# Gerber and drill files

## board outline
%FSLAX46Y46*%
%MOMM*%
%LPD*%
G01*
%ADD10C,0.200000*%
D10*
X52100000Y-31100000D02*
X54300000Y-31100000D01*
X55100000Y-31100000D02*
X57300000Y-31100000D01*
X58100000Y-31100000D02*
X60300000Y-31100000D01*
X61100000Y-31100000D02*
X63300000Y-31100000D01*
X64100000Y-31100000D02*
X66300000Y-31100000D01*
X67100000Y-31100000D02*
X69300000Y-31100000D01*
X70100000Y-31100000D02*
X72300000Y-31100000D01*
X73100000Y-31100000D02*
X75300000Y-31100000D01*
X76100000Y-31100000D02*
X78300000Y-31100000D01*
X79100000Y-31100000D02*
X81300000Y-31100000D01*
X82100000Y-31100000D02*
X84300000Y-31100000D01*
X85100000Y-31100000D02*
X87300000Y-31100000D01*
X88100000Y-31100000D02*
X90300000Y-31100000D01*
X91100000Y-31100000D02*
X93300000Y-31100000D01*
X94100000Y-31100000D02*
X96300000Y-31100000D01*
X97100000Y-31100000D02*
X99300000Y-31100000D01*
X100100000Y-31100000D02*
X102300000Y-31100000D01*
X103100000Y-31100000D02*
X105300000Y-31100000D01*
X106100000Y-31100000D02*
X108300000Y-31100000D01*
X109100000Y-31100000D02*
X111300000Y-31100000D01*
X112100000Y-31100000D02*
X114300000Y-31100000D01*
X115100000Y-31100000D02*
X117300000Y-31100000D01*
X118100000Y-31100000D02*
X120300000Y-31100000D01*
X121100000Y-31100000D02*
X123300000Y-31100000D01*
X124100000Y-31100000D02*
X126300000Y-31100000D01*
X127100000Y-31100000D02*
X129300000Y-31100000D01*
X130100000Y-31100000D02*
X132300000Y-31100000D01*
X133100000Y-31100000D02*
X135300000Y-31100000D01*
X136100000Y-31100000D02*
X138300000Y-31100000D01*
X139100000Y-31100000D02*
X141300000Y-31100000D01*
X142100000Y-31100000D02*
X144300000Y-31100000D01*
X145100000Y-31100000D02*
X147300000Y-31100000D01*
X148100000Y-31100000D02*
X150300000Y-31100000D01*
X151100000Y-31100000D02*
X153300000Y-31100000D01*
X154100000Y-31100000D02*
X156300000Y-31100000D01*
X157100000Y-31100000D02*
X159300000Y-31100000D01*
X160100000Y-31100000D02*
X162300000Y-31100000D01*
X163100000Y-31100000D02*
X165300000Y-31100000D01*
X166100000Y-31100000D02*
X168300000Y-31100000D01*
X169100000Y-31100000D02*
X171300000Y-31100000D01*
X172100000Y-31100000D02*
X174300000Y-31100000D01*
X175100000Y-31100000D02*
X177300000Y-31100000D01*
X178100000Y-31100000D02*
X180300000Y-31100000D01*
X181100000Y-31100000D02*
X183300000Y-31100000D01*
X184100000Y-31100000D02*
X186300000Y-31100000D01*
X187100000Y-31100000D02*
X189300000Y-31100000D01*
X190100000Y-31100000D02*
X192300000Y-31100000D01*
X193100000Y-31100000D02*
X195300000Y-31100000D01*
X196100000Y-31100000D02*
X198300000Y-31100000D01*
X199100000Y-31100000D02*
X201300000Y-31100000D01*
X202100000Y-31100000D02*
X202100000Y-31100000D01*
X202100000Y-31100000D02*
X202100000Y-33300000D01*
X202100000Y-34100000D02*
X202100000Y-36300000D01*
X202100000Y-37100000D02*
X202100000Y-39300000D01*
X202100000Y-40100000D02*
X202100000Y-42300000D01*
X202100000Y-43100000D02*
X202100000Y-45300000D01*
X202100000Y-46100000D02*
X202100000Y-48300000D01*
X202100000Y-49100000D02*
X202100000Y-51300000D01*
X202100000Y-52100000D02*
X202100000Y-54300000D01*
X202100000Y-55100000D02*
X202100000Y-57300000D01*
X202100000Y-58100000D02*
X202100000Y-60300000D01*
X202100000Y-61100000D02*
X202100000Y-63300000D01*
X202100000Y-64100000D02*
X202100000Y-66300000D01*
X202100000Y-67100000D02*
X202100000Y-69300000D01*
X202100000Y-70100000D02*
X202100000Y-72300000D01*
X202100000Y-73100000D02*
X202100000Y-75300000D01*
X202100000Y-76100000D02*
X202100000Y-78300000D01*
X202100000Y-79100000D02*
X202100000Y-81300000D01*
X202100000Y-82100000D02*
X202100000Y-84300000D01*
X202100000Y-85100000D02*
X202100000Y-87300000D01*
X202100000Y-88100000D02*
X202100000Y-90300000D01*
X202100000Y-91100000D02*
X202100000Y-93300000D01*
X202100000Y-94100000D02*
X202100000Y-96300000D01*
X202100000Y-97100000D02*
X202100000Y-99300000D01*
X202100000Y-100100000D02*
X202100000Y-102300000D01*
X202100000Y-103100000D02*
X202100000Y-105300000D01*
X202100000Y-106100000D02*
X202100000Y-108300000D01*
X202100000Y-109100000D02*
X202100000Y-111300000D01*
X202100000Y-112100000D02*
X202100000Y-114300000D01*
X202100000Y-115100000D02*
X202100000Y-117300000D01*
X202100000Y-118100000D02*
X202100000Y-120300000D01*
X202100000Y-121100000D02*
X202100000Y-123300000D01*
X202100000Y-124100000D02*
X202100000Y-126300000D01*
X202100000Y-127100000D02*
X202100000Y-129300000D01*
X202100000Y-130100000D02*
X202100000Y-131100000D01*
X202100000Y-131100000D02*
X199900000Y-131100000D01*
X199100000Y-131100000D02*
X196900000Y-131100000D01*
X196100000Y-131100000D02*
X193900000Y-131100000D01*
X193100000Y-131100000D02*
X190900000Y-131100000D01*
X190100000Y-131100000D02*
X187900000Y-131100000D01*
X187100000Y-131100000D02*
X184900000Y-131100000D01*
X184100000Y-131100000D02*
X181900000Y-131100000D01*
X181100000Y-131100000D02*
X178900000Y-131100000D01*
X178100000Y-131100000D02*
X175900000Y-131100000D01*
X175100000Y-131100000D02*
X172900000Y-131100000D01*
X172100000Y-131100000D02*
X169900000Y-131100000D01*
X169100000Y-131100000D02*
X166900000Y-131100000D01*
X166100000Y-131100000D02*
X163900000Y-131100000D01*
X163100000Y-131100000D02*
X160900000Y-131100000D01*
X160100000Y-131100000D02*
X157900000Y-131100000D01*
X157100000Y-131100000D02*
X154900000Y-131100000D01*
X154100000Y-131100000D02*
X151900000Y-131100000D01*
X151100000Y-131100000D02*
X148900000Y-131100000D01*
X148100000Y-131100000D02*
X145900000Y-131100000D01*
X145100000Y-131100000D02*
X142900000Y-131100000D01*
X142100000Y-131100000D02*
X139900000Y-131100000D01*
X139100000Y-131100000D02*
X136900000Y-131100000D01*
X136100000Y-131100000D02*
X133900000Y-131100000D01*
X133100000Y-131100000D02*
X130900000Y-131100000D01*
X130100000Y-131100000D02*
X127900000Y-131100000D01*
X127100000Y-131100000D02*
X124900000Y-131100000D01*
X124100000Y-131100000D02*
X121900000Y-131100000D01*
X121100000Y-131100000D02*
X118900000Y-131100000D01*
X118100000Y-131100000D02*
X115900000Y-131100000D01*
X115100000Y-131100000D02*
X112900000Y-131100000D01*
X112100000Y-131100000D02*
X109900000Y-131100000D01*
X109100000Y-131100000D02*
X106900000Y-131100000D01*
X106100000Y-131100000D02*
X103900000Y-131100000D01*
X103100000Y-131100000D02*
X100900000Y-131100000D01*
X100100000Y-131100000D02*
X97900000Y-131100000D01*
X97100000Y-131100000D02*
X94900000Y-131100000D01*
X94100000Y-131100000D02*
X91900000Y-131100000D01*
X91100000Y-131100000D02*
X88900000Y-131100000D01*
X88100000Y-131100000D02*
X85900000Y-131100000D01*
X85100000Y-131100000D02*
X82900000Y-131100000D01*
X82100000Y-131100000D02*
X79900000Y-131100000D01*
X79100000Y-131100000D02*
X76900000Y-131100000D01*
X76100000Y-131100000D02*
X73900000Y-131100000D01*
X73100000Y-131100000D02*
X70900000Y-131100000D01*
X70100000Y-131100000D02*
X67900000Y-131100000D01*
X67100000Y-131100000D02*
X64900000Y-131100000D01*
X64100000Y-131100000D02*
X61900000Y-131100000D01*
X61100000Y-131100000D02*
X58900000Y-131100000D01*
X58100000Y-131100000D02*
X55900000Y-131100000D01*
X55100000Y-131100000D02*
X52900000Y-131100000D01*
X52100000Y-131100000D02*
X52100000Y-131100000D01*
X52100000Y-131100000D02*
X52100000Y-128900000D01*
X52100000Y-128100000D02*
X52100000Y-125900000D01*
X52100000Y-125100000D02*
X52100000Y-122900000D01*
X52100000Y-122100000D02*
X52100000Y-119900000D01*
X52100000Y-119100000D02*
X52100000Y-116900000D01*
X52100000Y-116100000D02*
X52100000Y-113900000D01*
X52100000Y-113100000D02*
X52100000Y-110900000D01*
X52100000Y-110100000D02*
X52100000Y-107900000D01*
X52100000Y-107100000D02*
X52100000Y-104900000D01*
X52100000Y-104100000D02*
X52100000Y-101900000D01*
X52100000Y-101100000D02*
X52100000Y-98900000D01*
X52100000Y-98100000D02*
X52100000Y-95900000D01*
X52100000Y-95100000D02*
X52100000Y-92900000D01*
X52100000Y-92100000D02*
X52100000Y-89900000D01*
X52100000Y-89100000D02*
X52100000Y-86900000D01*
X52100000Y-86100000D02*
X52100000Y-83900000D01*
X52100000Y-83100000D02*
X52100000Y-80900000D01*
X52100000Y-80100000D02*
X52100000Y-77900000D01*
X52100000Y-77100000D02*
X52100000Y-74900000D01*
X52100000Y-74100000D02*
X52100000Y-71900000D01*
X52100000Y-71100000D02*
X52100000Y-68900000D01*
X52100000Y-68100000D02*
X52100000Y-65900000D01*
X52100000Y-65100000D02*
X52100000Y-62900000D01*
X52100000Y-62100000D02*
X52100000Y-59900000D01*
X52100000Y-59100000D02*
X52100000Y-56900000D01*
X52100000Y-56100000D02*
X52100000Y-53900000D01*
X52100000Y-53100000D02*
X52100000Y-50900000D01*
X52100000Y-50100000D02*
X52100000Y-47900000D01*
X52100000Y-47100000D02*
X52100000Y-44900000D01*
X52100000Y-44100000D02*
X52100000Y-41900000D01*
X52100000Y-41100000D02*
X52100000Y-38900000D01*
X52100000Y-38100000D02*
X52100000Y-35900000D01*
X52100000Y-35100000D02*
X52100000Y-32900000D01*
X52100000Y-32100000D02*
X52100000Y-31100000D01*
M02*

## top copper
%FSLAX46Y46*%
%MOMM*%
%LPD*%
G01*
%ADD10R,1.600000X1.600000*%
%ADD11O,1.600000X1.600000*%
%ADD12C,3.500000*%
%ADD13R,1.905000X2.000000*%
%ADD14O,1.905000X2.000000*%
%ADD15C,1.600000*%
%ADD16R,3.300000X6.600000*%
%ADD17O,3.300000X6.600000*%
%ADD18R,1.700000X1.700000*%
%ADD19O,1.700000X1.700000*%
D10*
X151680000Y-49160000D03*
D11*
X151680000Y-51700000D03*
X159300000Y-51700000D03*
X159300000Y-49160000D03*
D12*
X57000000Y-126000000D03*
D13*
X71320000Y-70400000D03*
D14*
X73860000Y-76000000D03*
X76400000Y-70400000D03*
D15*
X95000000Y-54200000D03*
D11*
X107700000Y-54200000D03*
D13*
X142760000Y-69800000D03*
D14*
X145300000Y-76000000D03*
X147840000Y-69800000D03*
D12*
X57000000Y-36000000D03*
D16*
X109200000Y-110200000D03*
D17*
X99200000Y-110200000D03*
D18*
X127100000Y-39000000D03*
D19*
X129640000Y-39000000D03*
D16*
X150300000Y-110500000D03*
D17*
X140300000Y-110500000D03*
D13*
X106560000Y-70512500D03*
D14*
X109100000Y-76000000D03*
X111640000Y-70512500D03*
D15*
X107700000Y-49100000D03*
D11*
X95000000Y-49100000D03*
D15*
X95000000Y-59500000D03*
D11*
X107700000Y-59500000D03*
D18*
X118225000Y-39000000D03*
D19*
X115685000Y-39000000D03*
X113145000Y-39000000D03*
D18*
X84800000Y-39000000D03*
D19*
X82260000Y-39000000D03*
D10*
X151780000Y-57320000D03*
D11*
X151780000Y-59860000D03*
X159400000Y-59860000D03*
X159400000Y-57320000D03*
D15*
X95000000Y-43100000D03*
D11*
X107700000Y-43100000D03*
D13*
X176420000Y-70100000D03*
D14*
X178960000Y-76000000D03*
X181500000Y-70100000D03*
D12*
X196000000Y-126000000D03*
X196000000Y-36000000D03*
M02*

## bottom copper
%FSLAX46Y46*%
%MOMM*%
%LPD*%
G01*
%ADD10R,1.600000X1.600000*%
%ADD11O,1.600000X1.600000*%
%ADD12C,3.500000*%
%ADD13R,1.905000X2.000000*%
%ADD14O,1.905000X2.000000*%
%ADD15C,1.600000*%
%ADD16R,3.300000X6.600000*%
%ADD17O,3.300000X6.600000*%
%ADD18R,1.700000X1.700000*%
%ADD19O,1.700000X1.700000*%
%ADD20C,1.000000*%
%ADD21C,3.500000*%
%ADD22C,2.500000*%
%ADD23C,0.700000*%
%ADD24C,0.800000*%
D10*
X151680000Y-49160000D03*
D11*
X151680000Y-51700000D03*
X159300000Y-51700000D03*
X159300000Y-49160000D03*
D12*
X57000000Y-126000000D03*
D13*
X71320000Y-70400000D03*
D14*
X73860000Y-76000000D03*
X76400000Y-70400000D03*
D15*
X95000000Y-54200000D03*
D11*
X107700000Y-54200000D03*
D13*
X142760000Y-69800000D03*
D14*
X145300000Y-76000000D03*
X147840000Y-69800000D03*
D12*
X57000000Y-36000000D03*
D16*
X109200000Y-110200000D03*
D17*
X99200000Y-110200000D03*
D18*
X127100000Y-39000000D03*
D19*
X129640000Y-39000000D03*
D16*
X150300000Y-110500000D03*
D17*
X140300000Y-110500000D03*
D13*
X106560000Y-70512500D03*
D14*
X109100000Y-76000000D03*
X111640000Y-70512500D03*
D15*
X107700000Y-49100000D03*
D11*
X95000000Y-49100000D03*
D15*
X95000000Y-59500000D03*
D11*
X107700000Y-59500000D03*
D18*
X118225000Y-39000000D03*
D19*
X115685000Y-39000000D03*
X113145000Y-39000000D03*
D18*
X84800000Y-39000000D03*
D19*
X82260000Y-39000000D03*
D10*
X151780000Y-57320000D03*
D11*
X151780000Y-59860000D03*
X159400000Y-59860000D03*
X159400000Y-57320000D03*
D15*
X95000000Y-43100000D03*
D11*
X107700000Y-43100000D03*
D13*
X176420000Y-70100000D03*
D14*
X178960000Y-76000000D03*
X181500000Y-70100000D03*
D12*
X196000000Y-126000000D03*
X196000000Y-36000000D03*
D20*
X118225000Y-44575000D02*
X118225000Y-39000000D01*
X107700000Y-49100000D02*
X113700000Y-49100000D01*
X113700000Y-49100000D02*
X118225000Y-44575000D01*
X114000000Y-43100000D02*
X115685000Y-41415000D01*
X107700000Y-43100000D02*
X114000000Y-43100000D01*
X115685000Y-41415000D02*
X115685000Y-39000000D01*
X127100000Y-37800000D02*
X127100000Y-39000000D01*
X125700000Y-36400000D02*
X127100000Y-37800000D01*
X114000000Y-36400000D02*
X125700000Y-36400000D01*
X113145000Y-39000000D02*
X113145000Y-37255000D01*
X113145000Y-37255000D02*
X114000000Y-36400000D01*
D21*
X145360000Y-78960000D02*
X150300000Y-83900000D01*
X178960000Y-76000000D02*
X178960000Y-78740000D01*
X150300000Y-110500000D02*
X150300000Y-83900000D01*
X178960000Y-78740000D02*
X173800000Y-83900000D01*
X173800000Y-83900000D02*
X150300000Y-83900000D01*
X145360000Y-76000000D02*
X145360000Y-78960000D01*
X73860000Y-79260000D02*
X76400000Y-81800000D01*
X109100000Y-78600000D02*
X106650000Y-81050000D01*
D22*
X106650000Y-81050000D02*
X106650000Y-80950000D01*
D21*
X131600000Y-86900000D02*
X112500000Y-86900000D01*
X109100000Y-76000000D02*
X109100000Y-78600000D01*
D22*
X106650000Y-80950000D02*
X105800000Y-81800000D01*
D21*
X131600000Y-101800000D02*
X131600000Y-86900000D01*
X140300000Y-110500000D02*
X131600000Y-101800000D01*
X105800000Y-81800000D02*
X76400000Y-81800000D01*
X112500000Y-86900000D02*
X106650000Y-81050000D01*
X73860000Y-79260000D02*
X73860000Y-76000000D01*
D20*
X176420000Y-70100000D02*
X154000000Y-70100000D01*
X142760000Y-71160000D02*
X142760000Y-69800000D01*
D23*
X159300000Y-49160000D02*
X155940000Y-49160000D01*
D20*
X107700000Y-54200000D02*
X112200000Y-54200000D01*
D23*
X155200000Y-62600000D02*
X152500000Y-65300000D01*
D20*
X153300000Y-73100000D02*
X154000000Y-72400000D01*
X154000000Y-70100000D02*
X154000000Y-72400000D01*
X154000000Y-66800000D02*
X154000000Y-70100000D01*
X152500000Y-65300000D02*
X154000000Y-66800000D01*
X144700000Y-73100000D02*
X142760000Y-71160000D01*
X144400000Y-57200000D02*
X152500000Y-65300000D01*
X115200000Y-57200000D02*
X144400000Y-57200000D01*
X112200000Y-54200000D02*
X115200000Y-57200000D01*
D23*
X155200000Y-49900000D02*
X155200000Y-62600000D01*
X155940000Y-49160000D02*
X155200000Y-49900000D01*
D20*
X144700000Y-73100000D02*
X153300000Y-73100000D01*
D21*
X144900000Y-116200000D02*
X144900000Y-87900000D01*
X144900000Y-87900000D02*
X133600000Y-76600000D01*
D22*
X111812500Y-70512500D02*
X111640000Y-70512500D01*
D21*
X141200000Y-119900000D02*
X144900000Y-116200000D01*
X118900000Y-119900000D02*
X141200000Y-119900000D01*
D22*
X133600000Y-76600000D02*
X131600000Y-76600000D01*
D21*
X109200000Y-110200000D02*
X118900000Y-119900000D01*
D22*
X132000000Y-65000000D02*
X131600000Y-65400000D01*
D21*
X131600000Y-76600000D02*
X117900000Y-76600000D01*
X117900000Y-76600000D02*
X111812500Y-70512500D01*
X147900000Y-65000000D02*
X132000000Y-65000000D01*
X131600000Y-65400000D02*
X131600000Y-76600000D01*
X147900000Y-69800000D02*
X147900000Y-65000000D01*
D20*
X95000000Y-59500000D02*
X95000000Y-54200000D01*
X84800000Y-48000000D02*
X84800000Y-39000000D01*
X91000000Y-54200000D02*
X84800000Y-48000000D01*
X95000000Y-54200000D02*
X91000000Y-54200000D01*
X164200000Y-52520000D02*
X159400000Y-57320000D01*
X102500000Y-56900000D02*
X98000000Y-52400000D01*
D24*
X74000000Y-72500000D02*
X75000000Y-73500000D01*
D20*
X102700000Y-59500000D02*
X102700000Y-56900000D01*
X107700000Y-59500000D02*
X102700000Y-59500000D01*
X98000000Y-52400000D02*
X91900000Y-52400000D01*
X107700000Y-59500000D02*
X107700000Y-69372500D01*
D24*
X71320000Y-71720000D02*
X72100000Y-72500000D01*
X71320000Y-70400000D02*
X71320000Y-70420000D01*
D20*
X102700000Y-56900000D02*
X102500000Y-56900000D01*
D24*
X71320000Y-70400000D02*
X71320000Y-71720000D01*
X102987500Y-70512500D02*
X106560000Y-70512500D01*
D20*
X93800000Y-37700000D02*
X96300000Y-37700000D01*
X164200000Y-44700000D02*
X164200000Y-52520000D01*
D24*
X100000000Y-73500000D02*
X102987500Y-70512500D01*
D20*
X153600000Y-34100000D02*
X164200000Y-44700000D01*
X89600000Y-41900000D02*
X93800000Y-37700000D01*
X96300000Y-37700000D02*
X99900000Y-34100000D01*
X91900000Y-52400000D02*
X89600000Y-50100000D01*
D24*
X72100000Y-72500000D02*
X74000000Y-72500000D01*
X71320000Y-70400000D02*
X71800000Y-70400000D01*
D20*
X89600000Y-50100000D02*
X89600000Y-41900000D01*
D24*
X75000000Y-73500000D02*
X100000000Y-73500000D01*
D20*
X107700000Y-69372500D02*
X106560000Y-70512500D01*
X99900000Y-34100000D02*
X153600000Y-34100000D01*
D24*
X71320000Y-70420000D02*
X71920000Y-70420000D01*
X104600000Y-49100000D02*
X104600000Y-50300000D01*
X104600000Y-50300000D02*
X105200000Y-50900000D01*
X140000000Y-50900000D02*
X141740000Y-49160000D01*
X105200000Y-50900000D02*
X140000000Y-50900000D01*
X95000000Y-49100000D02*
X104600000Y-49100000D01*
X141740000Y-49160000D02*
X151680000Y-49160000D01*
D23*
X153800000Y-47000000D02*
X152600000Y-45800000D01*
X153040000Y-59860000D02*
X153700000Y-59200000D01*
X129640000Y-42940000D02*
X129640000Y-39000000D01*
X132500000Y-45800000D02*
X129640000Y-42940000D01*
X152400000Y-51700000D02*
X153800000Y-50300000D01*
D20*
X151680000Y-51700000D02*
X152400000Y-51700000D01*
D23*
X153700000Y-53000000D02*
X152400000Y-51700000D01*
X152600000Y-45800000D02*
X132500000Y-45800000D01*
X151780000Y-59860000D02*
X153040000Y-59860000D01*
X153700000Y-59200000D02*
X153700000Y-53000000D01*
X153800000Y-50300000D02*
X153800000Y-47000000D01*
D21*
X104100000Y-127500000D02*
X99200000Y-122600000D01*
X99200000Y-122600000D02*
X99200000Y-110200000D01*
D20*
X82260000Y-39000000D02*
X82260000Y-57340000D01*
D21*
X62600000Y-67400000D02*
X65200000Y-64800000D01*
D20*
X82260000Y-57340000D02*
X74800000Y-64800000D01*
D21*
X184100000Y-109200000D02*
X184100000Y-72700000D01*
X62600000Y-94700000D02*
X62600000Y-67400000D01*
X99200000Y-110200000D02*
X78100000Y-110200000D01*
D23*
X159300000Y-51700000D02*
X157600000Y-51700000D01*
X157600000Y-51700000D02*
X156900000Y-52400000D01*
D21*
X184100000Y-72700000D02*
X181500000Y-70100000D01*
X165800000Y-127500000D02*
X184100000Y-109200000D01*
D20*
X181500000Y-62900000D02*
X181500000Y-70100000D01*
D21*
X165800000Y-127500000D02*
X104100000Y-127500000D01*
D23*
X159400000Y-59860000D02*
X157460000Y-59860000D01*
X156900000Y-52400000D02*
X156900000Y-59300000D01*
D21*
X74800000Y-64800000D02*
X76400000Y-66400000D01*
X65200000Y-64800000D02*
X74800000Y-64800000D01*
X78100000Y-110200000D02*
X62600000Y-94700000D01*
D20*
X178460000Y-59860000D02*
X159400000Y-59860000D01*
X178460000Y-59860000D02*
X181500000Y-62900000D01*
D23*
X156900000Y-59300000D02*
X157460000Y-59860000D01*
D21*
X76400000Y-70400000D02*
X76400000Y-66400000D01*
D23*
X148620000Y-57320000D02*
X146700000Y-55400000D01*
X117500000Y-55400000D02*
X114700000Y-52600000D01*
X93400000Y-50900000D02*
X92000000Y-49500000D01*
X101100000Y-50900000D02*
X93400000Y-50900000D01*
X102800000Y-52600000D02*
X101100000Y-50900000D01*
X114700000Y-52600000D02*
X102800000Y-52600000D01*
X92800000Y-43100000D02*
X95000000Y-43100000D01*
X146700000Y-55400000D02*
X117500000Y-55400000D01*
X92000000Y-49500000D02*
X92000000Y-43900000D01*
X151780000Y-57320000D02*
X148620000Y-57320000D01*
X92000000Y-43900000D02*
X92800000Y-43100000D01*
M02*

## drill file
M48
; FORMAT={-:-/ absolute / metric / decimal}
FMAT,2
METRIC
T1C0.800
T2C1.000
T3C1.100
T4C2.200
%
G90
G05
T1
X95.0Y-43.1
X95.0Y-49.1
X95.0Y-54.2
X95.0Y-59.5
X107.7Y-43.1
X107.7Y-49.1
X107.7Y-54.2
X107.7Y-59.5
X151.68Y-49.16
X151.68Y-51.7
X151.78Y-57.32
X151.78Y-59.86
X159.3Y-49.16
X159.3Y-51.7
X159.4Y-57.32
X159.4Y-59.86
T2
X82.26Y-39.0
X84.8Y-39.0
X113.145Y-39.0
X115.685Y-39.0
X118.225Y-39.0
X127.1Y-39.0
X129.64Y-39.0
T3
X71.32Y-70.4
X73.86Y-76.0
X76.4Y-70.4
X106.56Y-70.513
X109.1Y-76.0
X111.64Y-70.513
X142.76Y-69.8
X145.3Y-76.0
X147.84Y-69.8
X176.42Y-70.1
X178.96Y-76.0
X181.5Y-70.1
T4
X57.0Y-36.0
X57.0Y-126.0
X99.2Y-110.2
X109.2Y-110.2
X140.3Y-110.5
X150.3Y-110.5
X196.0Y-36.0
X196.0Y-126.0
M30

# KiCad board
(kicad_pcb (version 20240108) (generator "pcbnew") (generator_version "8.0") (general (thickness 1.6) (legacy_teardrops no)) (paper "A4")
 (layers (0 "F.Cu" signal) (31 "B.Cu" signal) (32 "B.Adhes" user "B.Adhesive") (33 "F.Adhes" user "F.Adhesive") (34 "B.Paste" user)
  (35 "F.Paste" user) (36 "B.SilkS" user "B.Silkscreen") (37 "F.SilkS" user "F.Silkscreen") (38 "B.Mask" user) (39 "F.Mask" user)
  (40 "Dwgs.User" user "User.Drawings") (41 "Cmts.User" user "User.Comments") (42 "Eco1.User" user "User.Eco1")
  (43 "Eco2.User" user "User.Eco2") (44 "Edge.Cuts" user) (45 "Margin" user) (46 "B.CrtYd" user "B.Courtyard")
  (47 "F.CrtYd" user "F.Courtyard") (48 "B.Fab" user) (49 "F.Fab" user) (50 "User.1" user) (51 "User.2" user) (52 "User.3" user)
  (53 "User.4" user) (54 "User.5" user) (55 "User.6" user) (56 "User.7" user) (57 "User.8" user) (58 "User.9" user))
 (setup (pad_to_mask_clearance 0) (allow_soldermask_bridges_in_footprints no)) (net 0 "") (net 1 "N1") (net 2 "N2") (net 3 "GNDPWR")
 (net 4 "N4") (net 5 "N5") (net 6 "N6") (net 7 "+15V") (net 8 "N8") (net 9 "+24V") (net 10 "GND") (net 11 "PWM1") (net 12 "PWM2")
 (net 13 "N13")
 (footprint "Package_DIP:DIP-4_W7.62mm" (layer "F.Cu") (at 151.68 49.16)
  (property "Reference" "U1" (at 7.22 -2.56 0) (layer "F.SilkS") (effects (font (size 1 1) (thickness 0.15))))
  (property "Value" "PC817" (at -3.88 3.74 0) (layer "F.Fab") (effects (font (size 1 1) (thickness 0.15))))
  (pad "1" thru_hole rect (at 0 0) (size 1.6 1.6) (drill 0.8) (layers "*.Cu" "*.Mask") (remove_unused_layers no) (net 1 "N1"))
  (pad "2" thru_hole oval (at 0 2.54) (size 1.6 1.6) (drill 0.8) (layers "*.Cu" "*.Mask") (remove_unused_layers no) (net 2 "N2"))
  (pad "3" thru_hole oval (at 7.62 2.54) (size 1.6 1.6) (drill 0.8) (layers "*.Cu" "*.Mask") (remove_unused_layers no) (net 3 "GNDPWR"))
  (pad "4" thru_hole oval (at 7.62 0) (size 1.6 1.6) (drill 0.8) (layers "*.Cu" "*.Mask") (remove_unused_layers no) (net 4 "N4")))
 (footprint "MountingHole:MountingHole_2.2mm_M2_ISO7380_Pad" (layer "F.Cu") (at 57 126)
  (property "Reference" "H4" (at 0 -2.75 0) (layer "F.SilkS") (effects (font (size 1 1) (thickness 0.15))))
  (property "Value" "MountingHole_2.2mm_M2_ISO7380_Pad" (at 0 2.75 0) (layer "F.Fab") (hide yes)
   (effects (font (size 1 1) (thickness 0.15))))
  (pad "1" thru_hole circle (at 0 0) (size 3.5 3.5) (drill 2.2) (layers "*.Cu" "*.Mask") (remove_unused_layers no)))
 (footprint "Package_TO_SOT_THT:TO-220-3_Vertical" (layer "F.Cu") (at 71.32 70.4)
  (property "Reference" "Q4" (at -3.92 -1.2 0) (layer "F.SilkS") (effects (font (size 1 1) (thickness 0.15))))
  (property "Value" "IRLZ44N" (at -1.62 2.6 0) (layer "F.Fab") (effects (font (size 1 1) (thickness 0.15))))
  (pad "1" thru_hole rect (at 0 0) (size 1.905 2) (drill 1.1) (layers "*.Cu" "*.Mask") (remove_unused_layers no) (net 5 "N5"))
  (pad "2" thru_hole oval (at 2.54 5.6) (size 1.905 2) (drill 1.1) (layers "*.Cu" "*.Mask") (remove_unused_layers no) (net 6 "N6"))
  (pad "3" thru_hole oval (at 5.08 0) (size 1.905 2) (drill 1.1) (layers "*.Cu" "*.Mask") (remove_unused_layers no) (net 3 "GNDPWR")))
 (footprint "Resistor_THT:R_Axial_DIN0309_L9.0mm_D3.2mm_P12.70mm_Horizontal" (layer "F.Cu") (at 95 54.2)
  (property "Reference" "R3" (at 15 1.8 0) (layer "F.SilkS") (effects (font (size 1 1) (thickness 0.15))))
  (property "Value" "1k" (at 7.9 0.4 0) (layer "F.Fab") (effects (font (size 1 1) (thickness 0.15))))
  (pad "1" thru_hole circle (at 0 0) (size 1.6 1.6) (drill 0.8) (layers "*.Cu" "*.Mask") (remove_unused_layers no) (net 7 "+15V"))
  (pad "2" thru_hole oval (at 12.7 0) (size 1.6 1.6) (drill 0.8) (layers "*.Cu" "*.Mask") (remove_unused_layers no) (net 4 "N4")))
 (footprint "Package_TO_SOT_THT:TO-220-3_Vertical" (layer "F.Cu") (at 142.76 69.8)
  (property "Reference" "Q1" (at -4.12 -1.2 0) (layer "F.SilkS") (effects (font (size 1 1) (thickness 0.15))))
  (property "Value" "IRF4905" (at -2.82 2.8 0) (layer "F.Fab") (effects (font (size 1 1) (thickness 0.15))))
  (pad "1" thru_hole rect (at 0 0) (size 1.905 2) (drill 1.1) (layers "*.Cu" "*.Mask") (remove_unused_layers no) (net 4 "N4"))
  (pad "2" thru_hole oval (at 2.54 6.2) (size 1.905 2) (drill 1.1) (layers "*.Cu" "*.Mask") (remove_unused_layers no) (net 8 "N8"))
  (pad "3" thru_hole oval (at 5.08 0) (size 1.905 2) (drill 1.1) (layers "*.Cu" "*.Mask") (remove_unused_layers no) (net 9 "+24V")))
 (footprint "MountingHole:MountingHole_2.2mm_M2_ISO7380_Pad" (layer "F.Cu") (at 57 36)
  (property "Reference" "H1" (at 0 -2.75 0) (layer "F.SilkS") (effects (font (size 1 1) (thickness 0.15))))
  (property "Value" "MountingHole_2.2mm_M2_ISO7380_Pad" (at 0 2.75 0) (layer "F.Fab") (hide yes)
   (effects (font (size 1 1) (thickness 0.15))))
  (pad "1" thru_hole circle (at 0 0) (size 3.5 3.5) (drill 2.2) (layers "*.Cu" "*.Mask") (remove_unused_layers no)))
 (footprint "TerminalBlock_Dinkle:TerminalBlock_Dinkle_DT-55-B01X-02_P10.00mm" (layer "F.Cu") (at 109.2 110.2 180)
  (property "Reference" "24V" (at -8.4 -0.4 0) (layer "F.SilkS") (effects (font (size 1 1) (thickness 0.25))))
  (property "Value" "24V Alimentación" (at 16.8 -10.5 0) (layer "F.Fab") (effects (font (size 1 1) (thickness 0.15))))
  (pad "1" thru_hole rect (at 0 0 180) (size 3.3 6.6) (drill 2.2) (layers "*.Cu" "*.Mask") (remove_unused_layers no) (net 9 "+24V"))
  (pad "2" thru_hole oval (at 10 0 180) (size 3.3 6.6) (drill 2.2) (layers "*.Cu" "*.Mask") (remove_unused_layers no) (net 3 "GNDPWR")))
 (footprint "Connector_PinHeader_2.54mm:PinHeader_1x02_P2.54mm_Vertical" (layer "F.Cu") (at 127.1 39 90)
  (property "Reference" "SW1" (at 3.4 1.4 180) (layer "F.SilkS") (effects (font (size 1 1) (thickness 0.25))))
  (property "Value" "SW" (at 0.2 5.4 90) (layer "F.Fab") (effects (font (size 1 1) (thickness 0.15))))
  (pad "1" thru_hole rect (at 0 0 90) (size 1.7 1.7) (drill 1) (layers "*.Cu" "*.Mask") (remove_unused_layers no) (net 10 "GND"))
  (pad "2" thru_hole oval (at 0 2.54 90) (size 1.7 1.7) (drill 1) (layers "*.Cu" "*.Mask") (remove_unused_layers no) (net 2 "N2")))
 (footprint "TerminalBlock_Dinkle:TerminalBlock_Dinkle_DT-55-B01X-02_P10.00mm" (layer "F.Cu") (at 150.3 110.5 180)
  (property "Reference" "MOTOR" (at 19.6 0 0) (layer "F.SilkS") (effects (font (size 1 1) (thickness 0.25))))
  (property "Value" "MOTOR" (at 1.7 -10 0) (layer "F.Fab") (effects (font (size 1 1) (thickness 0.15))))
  (pad "1" thru_hole rect (at 0 0 180) (size 3.3 6.6) (drill 2.2) (layers "*.Cu" "*.Mask") (remove_unused_layers no) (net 8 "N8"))
  (pad "2" thru_hole oval (at 10 0 180) (size 3.3 6.6) (drill 2.2) (layers "*.Cu" "*.Mask") (remove_unused_layers no) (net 6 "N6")))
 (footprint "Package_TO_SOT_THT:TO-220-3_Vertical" (layer "F.Cu") (at 106.56 70.5125)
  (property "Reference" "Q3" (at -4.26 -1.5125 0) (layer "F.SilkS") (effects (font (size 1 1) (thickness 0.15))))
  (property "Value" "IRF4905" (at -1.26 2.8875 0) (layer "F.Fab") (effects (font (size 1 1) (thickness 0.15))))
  (pad "1" thru_hole rect (at 0 0) (size 1.905 2) (drill 1.1) (layers "*.Cu" "*.Mask") (remove_unused_layers no) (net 5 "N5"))
  (pad "2" thru_hole oval (at 2.54 5.4875) (size 1.905 2) (drill 1.1) (layers "*.Cu" "*.Mask") (remove_unused_layers no) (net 6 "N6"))
  (pad "3" thru_hole oval (at 5.08 0) (size 1.905 2) (drill 1.1) (layers "*.Cu" "*.Mask") (remove_unused_layers no) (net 9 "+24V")))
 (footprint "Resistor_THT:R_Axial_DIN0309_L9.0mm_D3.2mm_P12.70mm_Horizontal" (layer "F.Cu") (at 107.7 49.1 180)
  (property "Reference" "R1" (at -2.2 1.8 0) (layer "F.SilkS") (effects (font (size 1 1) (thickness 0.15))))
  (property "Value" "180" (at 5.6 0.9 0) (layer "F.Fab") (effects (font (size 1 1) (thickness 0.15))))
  (pad "1" thru_hole circle (at 0 0 180) (size 1.6 1.6) (drill 0.8) (layers "*.Cu" "*.Mask") (remove_unused_layers no) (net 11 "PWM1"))
  (pad "2" thru_hole oval (at 12.7 0 180) (size 1.6 1.6) (drill 0.8) (layers "*.Cu" "*.Mask") (remove_unused_layers no) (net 1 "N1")))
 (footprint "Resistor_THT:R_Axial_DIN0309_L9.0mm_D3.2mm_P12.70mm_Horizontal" (layer "F.Cu") (at 95 59.5)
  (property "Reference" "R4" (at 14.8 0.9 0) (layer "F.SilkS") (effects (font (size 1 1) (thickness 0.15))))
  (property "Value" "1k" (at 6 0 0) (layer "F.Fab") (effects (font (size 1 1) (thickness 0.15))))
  (pad "1" thru_hole circle (at 0 0) (size 1.6 1.6) (drill 0.8) (layers "*.Cu" "*.Mask") (remove_unused_layers no) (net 7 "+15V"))
  (pad "2" thru_hole oval (at 12.7 0) (size 1.6 1.6) (drill 0.8) (layers "*.Cu" "*.Mask") (remove_unused_layers no) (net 5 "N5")))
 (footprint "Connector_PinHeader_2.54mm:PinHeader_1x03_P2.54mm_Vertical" (layer "F.Cu") (at 118.225 39 -90)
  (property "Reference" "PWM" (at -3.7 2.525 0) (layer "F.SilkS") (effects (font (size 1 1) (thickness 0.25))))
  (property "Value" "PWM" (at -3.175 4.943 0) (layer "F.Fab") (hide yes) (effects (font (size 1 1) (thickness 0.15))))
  (pad "1" thru_hole rect (at 0 0 270) (size 1.7 1.7) (drill 1) (layers "*.Cu" "*.Mask") (remove_unused_layers no) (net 11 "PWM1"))
  (pad "2" thru_hole oval (at 0 2.54 270) (size 1.7 1.7) (drill 1) (layers "*.Cu" "*.Mask") (remove_unused_layers no) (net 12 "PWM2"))
  (pad "3" thru_hole oval (at 0 5.08 270) (size 1.7 1.7) (drill 1) (layers "*.Cu" "*.Mask") (remove_unused_layers no) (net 10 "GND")))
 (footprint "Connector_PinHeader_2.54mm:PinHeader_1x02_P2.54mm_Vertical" (layer "F.Cu") (at 84.8 39 -90)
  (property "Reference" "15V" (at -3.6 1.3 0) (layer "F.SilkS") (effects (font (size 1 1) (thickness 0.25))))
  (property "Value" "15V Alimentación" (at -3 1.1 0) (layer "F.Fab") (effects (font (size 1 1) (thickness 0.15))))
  (pad "1" thru_hole rect (at 0 0 270) (size 1.7 1.7) (drill 1) (layers "*.Cu" "*.Mask") (remove_unused_layers no) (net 7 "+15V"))
  (pad "2" thru_hole oval (at 0 2.54 270) (size 1.7 1.7) (drill 1) (layers "*.Cu" "*.Mask") (remove_unused_layers no) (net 3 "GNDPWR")))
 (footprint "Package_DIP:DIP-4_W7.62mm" (layer "F.Cu") (at 151.78 57.32)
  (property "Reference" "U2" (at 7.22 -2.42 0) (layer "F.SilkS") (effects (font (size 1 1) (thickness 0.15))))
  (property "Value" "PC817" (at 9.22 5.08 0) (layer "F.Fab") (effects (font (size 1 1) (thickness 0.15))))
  (pad "1" thru_hole rect (at 0 0) (size 1.6 1.6) (drill 0.8) (layers "*.Cu" "*.Mask") (remove_unused_layers no) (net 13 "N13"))
  (pad "2" thru_hole oval (at 0 2.54) (size 1.6 1.6) (drill 0.8) (layers "*.Cu" "*.Mask") (remove_unused_layers no) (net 2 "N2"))
  (pad "3" thru_hole oval (at 7.62 2.54) (size 1.6 1.6) (drill 0.8) (layers "*.Cu" "*.Mask") (remove_unused_layers no) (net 3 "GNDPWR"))
  (pad "4" thru_hole oval (at 7.62 0) (size 1.6 1.6) (drill 0.8) (layers "*.Cu" "*.Mask") (remove_unused_layers no) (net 5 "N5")))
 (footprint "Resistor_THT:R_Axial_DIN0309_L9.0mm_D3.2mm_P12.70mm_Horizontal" (layer "F.Cu") (at 95 43.1)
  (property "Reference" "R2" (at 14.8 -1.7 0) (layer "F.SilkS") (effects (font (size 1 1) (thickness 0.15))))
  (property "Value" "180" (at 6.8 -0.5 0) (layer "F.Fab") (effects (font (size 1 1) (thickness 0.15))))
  (pad "1" thru_hole circle (at 0 0) (size 1.6 1.6) (drill 0.8) (layers "*.Cu" "*.Mask") (remove_unused_layers no) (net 13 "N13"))
  (pad "2" thru_hole oval (at 12.7 0) (size 1.6 1.6) (drill 0.8) (layers "*.Cu" "*.Mask") (remove_unused_layers no) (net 12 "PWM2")))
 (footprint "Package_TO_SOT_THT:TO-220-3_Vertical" (layer "F.Cu") (at 176.42 70.1)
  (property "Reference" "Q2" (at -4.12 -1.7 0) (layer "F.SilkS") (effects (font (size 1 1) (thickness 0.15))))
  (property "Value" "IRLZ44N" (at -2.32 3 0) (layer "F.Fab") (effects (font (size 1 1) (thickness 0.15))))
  (pad "1" thru_hole rect (at 0 0) (size 1.905 2) (drill 1.1) (layers "*.Cu" "*.Mask") (remove_unused_layers no) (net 4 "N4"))
  (pad "2" thru_hole oval (at 2.54 5.9) (size 1.905 2) (drill 1.1) (layers "*.Cu" "*.Mask") (remove_unused_layers no) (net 8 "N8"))
  (pad "3" thru_hole oval (at 5.08 0) (size 1.905 2) (drill 1.1) (layers "*.Cu" "*.Mask") (remove_unused_layers no) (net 3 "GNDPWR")))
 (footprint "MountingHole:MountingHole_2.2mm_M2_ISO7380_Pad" (layer "F.Cu") (at 196 126)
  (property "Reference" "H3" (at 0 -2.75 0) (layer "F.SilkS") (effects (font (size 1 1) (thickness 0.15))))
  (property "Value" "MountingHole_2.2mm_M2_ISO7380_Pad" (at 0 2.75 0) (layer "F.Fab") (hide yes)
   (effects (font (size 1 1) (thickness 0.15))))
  (pad "1" thru_hole circle (at 0 0) (size 3.5 3.5) (drill 2.2) (layers "*.Cu" "*.Mask") (remove_unused_layers no)))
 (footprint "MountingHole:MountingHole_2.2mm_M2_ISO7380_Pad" (layer "F.Cu") (at 196 36)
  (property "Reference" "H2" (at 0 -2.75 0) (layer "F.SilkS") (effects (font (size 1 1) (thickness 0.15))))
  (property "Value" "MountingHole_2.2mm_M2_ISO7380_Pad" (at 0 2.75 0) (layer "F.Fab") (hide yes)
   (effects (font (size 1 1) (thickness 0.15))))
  (pad "1" thru_hole circle (at 0 0) (size 3.5 3.5) (drill 2.2) (layers "*.Cu" "*.Mask") (remove_unused_layers no)))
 (gr_rect (start 52.1 31.1) (end 202.1 131.1) (stroke (width 0.2) (type dash)) (fill none) (layer "Edge.Cuts"))
 (segment (start 118.225 44.575) (end 118.225 39) (width 1) (layer "B.Cu") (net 11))
 (segment (start 107.7 49.1) (end 113.7 49.1) (width 1) (layer "B.Cu") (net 11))
 (segment (start 113.7 49.1) (end 118.225 44.575) (width 1) (layer "B.Cu") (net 11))
 (segment (start 114 43.1) (end 115.685 41.415) (width 1) (layer "B.Cu") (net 12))
 (segment (start 107.7 43.1) (end 114 43.1) (width 1) (layer "B.Cu") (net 12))
 (segment (start 115.685 41.415) (end 115.685 39) (width 1) (layer "B.Cu") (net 12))
 (segment (start 127.1 37.8) (end 127.1 39) (width 1) (layer "B.Cu") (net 10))
 (segment (start 125.7 36.4) (end 127.1 37.8) (width 1) (layer "B.Cu") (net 10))
 (segment (start 114 36.4) (end 125.7 36.4) (width 1) (layer "B.Cu") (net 10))
 (segment (start 113.145 39) (end 113.145 37.255) (width 1) (layer "B.Cu") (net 10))
 (segment (start 113.145 37.255) (end 114 36.4) (width 1) (layer "B.Cu") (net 10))
 (segment (start 145.36 78.96) (end 150.3 83.9) (width 3.5) (layer "B.Cu") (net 8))
 (segment (start 178.96 76) (end 178.96 78.74) (width 3.5) (layer "B.Cu") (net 8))
 (segment (start 150.3 110.5) (end 150.3 83.9) (width 3.5) (layer "B.Cu") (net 8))
 (segment (start 178.96 78.74) (end 173.8 83.9) (width 3.5) (layer "B.Cu") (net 8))
 (segment (start 173.8 83.9) (end 150.3 83.9) (width 3.5) (layer "B.Cu") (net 8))
 (segment (start 145.36 76) (end 145.36 78.96) (width 3.5) (layer "B.Cu") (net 8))
 (segment (start 73.86 79.26) (end 76.4 81.8) (width 3.5) (layer "B.Cu") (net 6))
 (segment (start 109.1 78.6) (end 106.65 81.05) (width 3.5) (layer "B.Cu") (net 6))
 (segment (start 106.65 81.05) (end 106.65 80.95) (width 2.5) (layer "B.Cu") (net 6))
 (segment (start 131.6 86.9) (end 112.5 86.9) (width 3.5) (layer "B.Cu") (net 6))
 (segment (start 109.1 76) (end 109.1 78.6) (width 3.5) (layer "B.Cu") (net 6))
 (segment (start 106.65 80.95) (end 105.8 81.8) (width 2.5) (layer "B.Cu") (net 6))
 (segment (start 131.6 101.8) (end 131.6 86.9) (width 3.5) (layer "B.Cu") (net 6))
 (segment (start 140.3 110.5) (end 131.6 101.8) (width 3.5) (layer "B.Cu") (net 6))
 (segment (start 105.8 81.8) (end 76.4 81.8) (width 3.5) (layer "B.Cu") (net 6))
 (segment (start 112.5 86.9) (end 106.65 81.05) (width 3.5) (layer "B.Cu") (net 6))
 (segment (start 73.86 79.26) (end 73.86 76) (width 3.5) (layer "B.Cu") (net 6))
 (segment (start 176.42 70.1) (end 154 70.1) (width 1) (layer "B.Cu") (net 4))
 (segment (start 142.76 71.16) (end 142.76 69.8) (width 1) (layer "B.Cu") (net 4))
 (segment (start 159.3 49.16) (end 155.94 49.16) (width 0.7) (layer "B.Cu") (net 4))
 (segment (start 107.7 54.2) (end 112.2 54.2) (width 1) (layer "B.Cu") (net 4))
 (segment (start 155.2 62.6) (end 152.5 65.3) (width 0.7) (layer "B.Cu") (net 4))
 (segment (start 153.3 73.1) (end 154 72.4) (width 1) (layer "B.Cu") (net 4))
 (segment (start 154 70.1) (end 154 72.4) (width 1) (layer "B.Cu") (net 4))
 (segment (start 154 66.8) (end 154 70.1) (width 1) (layer "B.Cu") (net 4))
 (segment (start 152.5 65.3) (end 154 66.8) (width 1) (layer "B.Cu") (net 4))
 (segment (start 144.7 73.1) (end 142.76 71.16) (width 1) (layer "B.Cu") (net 4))
 (segment (start 144.4 57.2) (end 152.5 65.3) (width 1) (layer "B.Cu") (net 4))
 (segment (start 115.2 57.2) (end 144.4 57.2) (width 1) (layer "B.Cu") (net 4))
 (segment (start 112.2 54.2) (end 115.2 57.2) (width 1) (layer "B.Cu") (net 4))
 (segment (start 155.2 49.9) (end 155.2 62.6) (width 0.7) (layer "B.Cu") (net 4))
 (segment (start 155.94 49.16) (end 155.2 49.9) (width 0.7) (layer "B.Cu") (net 4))
 (segment (start 144.7 73.1) (end 153.3 73.1) (width 1) (layer "B.Cu") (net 4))
 (segment (start 144.9 116.2) (end 144.9 87.9) (width 3.5) (layer "B.Cu") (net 9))
 (segment (start 144.9 87.9) (end 133.6 76.6) (width 3.5) (layer "B.Cu") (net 9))
 (segment (start 111.8125 70.5125) (end 111.64 70.5125) (width 2.5) (layer "B.Cu") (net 9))
 (segment (start 141.2 119.9) (end 144.9 116.2) (width 3.5) (layer "B.Cu") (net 9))
 (segment (start 118.9 119.9) (end 141.2 119.9) (width 3.5) (layer "B.Cu") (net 9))
 (segment (start 133.6 76.6) (end 131.6 76.6) (width 2.5) (layer "B.Cu") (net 9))
 (segment (start 109.2 110.2) (end 118.9 119.9) (width 3.5) (layer "B.Cu") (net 9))
 (segment (start 132 65) (end 131.6 65.4) (width 2.5) (layer "B.Cu") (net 9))
 (segment (start 131.6 76.6) (end 117.9 76.6) (width 3.5) (layer "B.Cu") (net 9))
 (segment (start 117.9 76.6) (end 111.8125 70.5125) (width 3.5) (layer "B.Cu") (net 9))
 (segment (start 147.9 65) (end 132 65) (width 3.5) (layer "B.Cu") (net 9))
 (segment (start 131.6 65.4) (end 131.6 76.6) (width 3.5) (layer "B.Cu") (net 9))
 (segment (start 147.9 69.8) (end 147.9 65) (width 3.5) (layer "B.Cu") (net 9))
 (segment (start 95 59.5) (end 95 54.2) (width 1) (layer "B.Cu") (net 7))
 (segment (start 84.8 48) (end 84.8 39) (width 1) (layer "B.Cu") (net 7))
 (segment (start 91 54.2) (end 84.8 48) (width 1) (layer "B.Cu") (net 7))
 (segment (start 95 54.2) (end 91 54.2) (width 1) (layer "B.Cu") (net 7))
 (segment (start 164.2 52.52) (end 159.4 57.32) (width 1) (layer "B.Cu") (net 5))
 (segment (start 102.5 56.9) (end 98 52.4) (width 1) (layer "B.Cu") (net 5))
 (segment (start 74 72.5) (end 75 73.5) (width 0.8) (layer "B.Cu") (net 5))
 (segment (start 102.7 59.5) (end 102.7 56.9) (width 1) (layer "B.Cu") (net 5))
 (segment (start 107.7 59.5) (end 102.7 59.5) (width 1) (layer "B.Cu") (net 5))
 (segment (start 98 52.4) (end 91.9 52.4) (width 1) (layer "B.Cu") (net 5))
 (segment (start 107.7 59.5) (end 107.7 69.3725) (width 1) (layer "B.Cu") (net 5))
 (segment (start 71.32 71.72) (end 72.1 72.5) (width 0.8) (layer "B.Cu") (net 5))
 (segment (start 71.32 70.4) (end 71.32 70.42) (width 0.8) (layer "B.Cu") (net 5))
 (segment (start 102.7 56.9) (end 102.5 56.9) (width 1) (layer "B.Cu") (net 5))
 (segment (start 71.32 70.4) (end 71.32 71.72) (width 0.8) (layer "B.Cu") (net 5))
 (segment (start 102.9875 70.5125) (end 106.56 70.5125) (width 0.8) (layer "B.Cu") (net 5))
 (segment (start 93.8 37.7) (end 96.3 37.7) (width 1) (layer "B.Cu") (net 5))
 (segment (start 164.2 44.7) (end 164.2 52.52) (width 1) (layer "B.Cu") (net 5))
 (segment (start 100 73.5) (end 102.9875 70.5125) (width 0.8) (layer "B.Cu") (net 5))
 (segment (start 153.6 34.1) (end 164.2 44.7) (width 1) (layer "B.Cu") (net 5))
 (segment (start 89.6 41.9) (end 93.8 37.7) (width 1) (layer "B.Cu") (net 5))
 (segment (start 96.3 37.7) (end 99.9 34.1) (width 1) (layer "B.Cu") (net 5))
 (segment (start 91.9 52.4) (end 89.6 50.1) (width 1) (layer "B.Cu") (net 5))
 (segment (start 72.1 72.5) (end 74 72.5) (width 0.8) (layer "B.Cu") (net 5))
 (segment (start 71.32 70.4) (end 71.8 70.4) (width 0.8) (layer "B.Cu") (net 5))
 (segment (start 89.6 50.1) (end 89.6 41.9) (width 1) (layer "B.Cu") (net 5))
 (segment (start 75 73.5) (end 100 73.5) (width 0.8) (layer "B.Cu") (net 5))
 (segment (start 107.7 69.3725) (end 106.56 70.5125) (width 1) (layer "B.Cu") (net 5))
 (segment (start 99.9 34.1) (end 153.6 34.1) (width 1) (layer "B.Cu") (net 5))
 (segment (start 71.32 70.42) (end 71.92 70.42) (width 0.8) (layer "B.Cu") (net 5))
 (segment (start 104.6 49.1) (end 104.6 50.3) (width 0.8) (layer "B.Cu") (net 1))
 (segment (start 104.6 50.3) (end 105.2 50.9) (width 0.8) (layer "B.Cu") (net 1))
 (segment (start 140 50.9) (end 141.74 49.16) (width 0.8) (layer "B.Cu") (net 1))
 (segment (start 105.2 50.9) (end 140 50.9) (width 0.8) (layer "B.Cu") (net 1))
 (segment (start 95 49.1) (end 104.6 49.1) (width 0.8) (layer "B.Cu") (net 1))
 (segment (start 141.74 49.16) (end 151.68 49.16) (width 0.8) (layer "B.Cu") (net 1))
 (segment (start 153.8 47) (end 152.6 45.8) (width 0.7) (layer "B.Cu") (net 2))
 (segment (start 153.04 59.86) (end 153.7 59.2) (width 0.7) (layer "B.Cu") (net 2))
 (segment (start 129.64 42.94) (end 129.64 39) (width 0.7) (layer "B.Cu") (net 2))
 (segment (start 132.5 45.8) (end 129.64 42.94) (width 0.7) (layer "B.Cu") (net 2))
 (segment (start 152.4 51.7) (end 153.8 50.3) (width 0.7) (layer "B.Cu") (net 2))
 (segment (start 151.68 51.7) (end 152.4 51.7) (width 1) (layer "B.Cu") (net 2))
 (segment (start 153.7 53) (end 152.4 51.7) (width 0.7) (layer "B.Cu") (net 2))
 (segment (start 152.6 45.8) (end 132.5 45.8) (width 0.7) (layer "B.Cu") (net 2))
 (segment (start 151.78 59.86) (end 153.04 59.86) (width 0.7) (layer "B.Cu") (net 2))
 (segment (start 153.7 59.2) (end 153.7 53) (width 0.7) (layer "B.Cu") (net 2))
 (segment (start 153.8 50.3) (end 153.8 47) (width 0.7) (layer "B.Cu") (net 2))
 (segment (start 104.1 127.5) (end 99.2 122.6) (width 3.5) (layer "B.Cu") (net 3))
 (segment (start 99.2 122.6) (end 99.2 110.2) (width 3.5) (layer "B.Cu") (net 3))
 (segment (start 82.26 39) (end 82.26 57.34) (width 1) (layer "B.Cu") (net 3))
 (segment (start 62.6 67.4) (end 65.2 64.8) (width 3.5) (layer "B.Cu") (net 3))
 (segment (start 82.26 57.34) (end 74.8 64.8) (width 1) (layer "B.Cu") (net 3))
 (segment (start 184.1 109.2) (end 184.1 72.7) (width 3.5) (layer "B.Cu") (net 3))
 (segment (start 62.6 94.7) (end 62.6 67.4) (width 3.5) (layer "B.Cu") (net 3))
 (segment (start 99.2 110.2) (end 78.1 110.2) (width 3.5) (layer "B.Cu") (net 3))
 (segment (start 159.3 51.7) (end 157.6 51.7) (width 0.7) (layer "B.Cu") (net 3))
 (segment (start 157.6 51.7) (end 156.9 52.4) (width 0.7) (layer "B.Cu") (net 3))
 (segment (start 184.1 72.7) (end 181.5 70.1) (width 3.5) (layer "B.Cu") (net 3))
 (segment (start 165.8 127.5) (end 184.1 109.2) (width 3.5) (layer "B.Cu") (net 3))
 (segment (start 181.5 62.9) (end 181.5 70.1) (width 1) (layer "B.Cu") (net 3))
 (segment (start 165.8 127.5) (end 104.1 127.5) (width 3.5) (layer "B.Cu") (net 3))
 (segment (start 159.4 59.86) (end 157.46 59.86) (width 0.7) (layer "B.Cu") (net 3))
 (segment (start 156.9 52.4) (end 156.9 59.3) (width 0.7) (layer "B.Cu") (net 3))
 (segment (start 74.8 64.8) (end 76.4 66.4) (width 3.5) (layer "B.Cu") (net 3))
 (segment (start 65.2 64.8) (end 74.8 64.8) (width 3.5) (layer "B.Cu") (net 3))
 (segment (start 78.1 110.2) (end 62.6 94.7) (width 3.5) (layer "B.Cu") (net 3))
 (segment (start 178.46 59.86) (end 159.4 59.86) (width 1) (layer "B.Cu") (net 3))
 (segment (start 178.46 59.86) (end 181.5 62.9) (width 1) (layer "B.Cu") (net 3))
 (segment (start 156.9 59.3) (end 157.46 59.86) (width 0.7) (layer "B.Cu") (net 3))
 (segment (start 76.4 70.4) (end 76.4 66.4) (width 3.5) (layer "B.Cu") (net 3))
 (segment (start 148.62 57.32) (end 146.7 55.4) (width 0.7) (layer "B.Cu") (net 13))
 (segment (start 117.5 55.4) (end 114.7 52.6) (width 0.7) (layer "B.Cu") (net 13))
 (segment (start 93.4 50.9) (end 92 49.5) (width 0.7) (layer "B.Cu") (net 13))
 (segment (start 101.1 50.9) (end 93.4 50.9) (width 0.7) (layer "B.Cu") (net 13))
 (segment (start 102.8 52.6) (end 101.1 50.9) (width 0.7) (layer "B.Cu") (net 13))
 (segment (start 114.7 52.6) (end 102.8 52.6) (width 0.7) (layer "B.Cu") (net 13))
 (segment (start 92.8 43.1) (end 95 43.1) (width 0.7) (layer "B.Cu") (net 13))
 (segment (start 146.7 55.4) (end 117.5 55.4) (width 0.7) (layer "B.Cu") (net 13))
 (segment (start 92 49.5) (end 92 43.9) (width 0.7) (layer "B.Cu") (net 13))
 (segment (start 151.78 57.32) (end 148.62 57.32) (width 0.7) (layer "B.Cu") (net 13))
 (segment (start 92 43.9) (end 92.8 43.1) (width 0.7) (layer "B.Cu") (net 13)))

